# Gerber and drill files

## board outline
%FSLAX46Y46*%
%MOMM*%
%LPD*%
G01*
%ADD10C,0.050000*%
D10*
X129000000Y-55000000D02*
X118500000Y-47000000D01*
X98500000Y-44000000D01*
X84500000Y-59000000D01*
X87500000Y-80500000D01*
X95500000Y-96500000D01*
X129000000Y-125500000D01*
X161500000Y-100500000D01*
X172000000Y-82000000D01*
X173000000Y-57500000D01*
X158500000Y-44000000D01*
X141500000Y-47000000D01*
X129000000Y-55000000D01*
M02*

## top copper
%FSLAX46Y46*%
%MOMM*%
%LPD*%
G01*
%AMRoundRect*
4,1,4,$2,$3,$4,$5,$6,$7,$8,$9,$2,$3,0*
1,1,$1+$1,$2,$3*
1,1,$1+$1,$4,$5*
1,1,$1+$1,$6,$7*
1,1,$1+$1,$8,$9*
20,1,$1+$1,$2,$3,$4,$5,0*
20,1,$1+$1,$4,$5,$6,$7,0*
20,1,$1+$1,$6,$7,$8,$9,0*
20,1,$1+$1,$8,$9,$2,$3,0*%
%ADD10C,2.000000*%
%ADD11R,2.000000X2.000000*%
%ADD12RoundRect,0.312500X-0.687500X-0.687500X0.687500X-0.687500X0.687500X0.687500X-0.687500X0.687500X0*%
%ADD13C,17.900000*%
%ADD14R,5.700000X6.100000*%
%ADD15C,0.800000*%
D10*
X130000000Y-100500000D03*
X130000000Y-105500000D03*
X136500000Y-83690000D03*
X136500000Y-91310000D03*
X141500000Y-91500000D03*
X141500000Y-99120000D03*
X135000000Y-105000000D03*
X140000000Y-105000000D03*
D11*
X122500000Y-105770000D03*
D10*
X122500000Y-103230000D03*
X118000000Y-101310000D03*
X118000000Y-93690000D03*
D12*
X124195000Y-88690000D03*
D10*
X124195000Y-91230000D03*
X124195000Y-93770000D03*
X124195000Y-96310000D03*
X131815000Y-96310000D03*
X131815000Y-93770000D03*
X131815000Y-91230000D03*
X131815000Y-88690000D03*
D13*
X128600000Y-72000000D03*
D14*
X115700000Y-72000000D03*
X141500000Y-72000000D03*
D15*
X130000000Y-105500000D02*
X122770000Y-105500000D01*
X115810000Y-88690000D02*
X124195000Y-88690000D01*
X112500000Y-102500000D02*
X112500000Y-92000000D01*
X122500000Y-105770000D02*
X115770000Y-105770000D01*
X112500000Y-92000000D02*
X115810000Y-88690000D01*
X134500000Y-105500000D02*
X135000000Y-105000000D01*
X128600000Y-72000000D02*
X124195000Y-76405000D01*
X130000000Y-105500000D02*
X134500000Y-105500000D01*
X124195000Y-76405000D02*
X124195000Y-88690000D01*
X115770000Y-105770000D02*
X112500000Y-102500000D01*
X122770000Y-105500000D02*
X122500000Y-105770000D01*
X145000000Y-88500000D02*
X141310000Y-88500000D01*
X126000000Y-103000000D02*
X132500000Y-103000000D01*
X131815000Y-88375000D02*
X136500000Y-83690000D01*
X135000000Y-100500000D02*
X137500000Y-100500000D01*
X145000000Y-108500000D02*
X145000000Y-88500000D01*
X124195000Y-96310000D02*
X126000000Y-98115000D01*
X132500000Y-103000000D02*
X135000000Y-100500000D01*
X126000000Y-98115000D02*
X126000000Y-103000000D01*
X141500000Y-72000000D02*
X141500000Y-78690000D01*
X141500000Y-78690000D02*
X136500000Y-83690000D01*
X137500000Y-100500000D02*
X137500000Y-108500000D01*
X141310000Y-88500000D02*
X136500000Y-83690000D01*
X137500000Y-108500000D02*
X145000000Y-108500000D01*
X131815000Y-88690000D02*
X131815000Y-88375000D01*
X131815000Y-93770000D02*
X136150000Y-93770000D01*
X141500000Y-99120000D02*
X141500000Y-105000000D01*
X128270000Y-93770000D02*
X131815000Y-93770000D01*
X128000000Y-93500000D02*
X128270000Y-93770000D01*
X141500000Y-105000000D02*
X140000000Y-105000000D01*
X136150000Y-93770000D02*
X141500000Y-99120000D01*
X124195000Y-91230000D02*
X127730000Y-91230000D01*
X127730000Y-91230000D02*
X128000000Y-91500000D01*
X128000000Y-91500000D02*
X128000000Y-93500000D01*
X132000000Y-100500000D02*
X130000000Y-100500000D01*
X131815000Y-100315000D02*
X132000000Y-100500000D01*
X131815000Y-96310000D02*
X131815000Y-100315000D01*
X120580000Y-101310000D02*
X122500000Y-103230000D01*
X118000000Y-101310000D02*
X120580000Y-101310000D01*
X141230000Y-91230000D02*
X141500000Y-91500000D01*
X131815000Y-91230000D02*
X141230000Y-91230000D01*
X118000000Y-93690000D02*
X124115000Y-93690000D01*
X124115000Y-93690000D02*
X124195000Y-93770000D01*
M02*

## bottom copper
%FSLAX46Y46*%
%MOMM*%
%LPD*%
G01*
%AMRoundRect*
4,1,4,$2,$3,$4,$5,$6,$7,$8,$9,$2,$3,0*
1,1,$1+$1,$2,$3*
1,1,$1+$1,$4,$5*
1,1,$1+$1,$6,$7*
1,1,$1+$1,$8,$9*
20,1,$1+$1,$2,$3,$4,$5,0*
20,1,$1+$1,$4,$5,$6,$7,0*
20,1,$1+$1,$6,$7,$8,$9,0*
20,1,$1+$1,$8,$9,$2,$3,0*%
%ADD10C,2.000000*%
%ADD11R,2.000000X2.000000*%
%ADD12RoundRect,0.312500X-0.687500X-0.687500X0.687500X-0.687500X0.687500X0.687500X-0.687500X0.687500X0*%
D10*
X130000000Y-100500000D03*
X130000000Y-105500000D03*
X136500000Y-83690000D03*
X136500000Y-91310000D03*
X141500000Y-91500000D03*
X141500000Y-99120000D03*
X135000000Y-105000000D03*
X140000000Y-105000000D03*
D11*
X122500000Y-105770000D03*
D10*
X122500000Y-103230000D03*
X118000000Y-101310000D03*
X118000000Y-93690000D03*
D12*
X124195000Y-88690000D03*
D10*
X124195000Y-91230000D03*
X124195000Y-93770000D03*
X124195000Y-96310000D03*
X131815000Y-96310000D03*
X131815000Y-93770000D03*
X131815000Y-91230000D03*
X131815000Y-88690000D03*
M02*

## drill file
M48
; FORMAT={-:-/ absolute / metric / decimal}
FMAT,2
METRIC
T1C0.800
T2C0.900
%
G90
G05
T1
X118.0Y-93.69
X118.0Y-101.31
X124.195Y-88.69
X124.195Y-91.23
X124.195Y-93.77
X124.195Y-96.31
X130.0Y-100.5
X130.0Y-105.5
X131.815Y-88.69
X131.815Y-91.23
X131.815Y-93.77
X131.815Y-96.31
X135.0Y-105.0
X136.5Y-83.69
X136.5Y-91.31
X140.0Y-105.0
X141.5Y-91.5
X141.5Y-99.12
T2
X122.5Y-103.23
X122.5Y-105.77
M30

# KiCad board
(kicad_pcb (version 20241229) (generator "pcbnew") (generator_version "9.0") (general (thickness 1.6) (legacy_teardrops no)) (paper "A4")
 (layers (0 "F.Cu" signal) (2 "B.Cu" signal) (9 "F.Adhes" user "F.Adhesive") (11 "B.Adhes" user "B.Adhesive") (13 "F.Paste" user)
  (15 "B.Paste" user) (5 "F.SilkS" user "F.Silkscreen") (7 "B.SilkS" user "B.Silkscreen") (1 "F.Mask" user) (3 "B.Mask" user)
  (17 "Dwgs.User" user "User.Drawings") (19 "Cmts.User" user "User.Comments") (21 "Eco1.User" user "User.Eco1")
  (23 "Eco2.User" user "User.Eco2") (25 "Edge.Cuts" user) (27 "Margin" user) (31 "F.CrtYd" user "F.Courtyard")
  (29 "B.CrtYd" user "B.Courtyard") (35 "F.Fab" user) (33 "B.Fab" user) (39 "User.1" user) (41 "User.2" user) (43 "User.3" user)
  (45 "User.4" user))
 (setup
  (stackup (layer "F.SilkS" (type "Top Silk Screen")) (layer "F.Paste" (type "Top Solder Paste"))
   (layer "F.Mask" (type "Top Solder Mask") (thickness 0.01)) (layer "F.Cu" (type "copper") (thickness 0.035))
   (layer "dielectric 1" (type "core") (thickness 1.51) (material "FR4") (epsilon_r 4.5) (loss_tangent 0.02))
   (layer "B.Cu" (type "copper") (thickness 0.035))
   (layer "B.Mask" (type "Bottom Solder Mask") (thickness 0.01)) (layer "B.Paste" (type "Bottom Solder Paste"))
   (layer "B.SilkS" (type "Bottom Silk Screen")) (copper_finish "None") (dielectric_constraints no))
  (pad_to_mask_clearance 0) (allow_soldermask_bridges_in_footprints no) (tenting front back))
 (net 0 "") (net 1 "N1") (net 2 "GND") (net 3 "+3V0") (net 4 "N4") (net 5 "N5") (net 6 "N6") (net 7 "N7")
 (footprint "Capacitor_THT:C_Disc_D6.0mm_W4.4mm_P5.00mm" (layer "F.Cu") (at 130 100.5 -90)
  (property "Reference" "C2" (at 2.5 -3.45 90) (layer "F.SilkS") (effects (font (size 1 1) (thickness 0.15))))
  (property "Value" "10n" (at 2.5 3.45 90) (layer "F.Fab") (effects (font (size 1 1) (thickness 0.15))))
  (pad "1" thru_hole circle (at 0 0 270) (size 2 2) (drill 0.8) (layers "*.Cu" "*.Mask") (remove_unused_layers no) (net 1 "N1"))
  (pad "2" thru_hole circle (at 5 0 270) (size 2 2) (drill 0.8) (layers "*.Cu" "*.Mask") (remove_unused_layers no) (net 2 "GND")))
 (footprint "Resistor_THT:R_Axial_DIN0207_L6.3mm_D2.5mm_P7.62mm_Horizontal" (layer "F.Cu") (at 136.5 83.69 -90)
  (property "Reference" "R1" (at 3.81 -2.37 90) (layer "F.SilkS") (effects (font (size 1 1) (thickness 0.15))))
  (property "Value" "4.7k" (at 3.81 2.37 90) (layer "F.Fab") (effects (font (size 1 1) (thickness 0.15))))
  (pad "1" thru_hole circle (at 0 0 270) (size 2 2) (drill 0.8) (layers "*.Cu" "*.Mask") (remove_unused_layers no) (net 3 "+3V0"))
  (pad "2" thru_hole circle (at 7.62 0 270) (size 2 2) (drill 0.8) (layers "*.Cu" "*.Mask") (remove_unused_layers no) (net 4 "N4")))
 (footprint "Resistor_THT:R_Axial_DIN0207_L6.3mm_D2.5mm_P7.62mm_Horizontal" (layer "F.Cu") (at 141.5 91.5 -90)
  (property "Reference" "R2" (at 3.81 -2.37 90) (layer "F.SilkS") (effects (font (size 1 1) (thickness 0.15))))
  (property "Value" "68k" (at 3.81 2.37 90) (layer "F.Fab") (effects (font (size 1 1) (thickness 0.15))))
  (pad "1" thru_hole circle (at 0 0 270) (size 2 2) (drill 0.8) (layers "*.Cu" "*.Mask") (remove_unused_layers no) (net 4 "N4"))
  (pad "2" thru_hole circle (at 7.62 0 270) (size 2 2) (drill 0.8) (layers "*.Cu" "*.Mask") (remove_unused_layers no) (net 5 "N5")))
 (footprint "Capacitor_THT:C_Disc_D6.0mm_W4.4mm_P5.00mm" (layer "F.Cu") (at 135 105)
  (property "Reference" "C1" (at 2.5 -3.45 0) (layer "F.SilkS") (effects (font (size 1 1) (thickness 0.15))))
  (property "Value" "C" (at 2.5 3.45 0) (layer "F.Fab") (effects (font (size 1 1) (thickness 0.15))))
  (pad "1" thru_hole circle (at 0 0) (size 2 2) (drill 0.8) (layers "*.Cu" "*.Mask") (remove_unused_layers no) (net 2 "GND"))
  (pad "2" thru_hole circle (at 5 0) (size 2 2) (drill 0.8) (layers "*.Cu" "*.Mask") (remove_unused_layers no) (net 5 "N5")))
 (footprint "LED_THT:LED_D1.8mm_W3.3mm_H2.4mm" (layer "F.Cu") (at 122.5 105.77 90)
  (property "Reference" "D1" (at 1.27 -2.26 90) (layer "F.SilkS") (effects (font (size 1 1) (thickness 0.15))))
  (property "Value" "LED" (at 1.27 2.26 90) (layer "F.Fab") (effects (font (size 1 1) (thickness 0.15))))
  (pad "1" thru_hole rect (at 0 0 90) (size 2 2) (drill 0.9) (layers "*.Cu" "*.Mask") (remove_unused_layers no) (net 2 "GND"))
  (pad "2" thru_hole circle (at 2.54 0 90) (size 2 2) (drill 0.9) (layers "*.Cu" "*.Mask") (remove_unused_layers no) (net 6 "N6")))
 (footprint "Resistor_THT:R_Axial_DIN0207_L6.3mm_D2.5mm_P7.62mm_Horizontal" (layer "F.Cu") (at 118 101.31 90)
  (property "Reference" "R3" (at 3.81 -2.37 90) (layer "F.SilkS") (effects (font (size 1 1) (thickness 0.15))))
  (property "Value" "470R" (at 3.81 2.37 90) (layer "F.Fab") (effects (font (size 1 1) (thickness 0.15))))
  (pad "1" thru_hole circle (at 0 0 90) (size 2 2) (drill 0.8) (layers "*.Cu" "*.Mask") (remove_unused_layers no) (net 6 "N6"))
  (pad "2" thru_hole circle (at 7.62 0 90) (size 2 2) (drill 0.8) (layers "*.Cu" "*.Mask") (remove_unused_layers no) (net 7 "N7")))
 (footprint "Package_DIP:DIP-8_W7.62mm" (layer "F.Cu") (at 124.195 88.69)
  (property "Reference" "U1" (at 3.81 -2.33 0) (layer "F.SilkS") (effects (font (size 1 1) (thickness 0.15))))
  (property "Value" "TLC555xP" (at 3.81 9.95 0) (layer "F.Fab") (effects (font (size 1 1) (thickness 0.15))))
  (pad "1" thru_hole roundrect (at 0 0) (size 2 2) (drill 0.8) (layers "*.Cu" "*.Mask") (remove_unused_layers no) (roundrect_rratio 0.15625)
   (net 2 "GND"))
  (pad "2" thru_hole circle (at 0 2.54) (size 2 2) (drill 0.8) (layers "*.Cu" "*.Mask") (remove_unused_layers no) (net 5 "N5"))
  (pad "3" thru_hole circle (at 0 5.08) (size 2 2) (drill 0.8) (layers "*.Cu" "*.Mask") (remove_unused_layers no) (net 7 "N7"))
  (pad "4" thru_hole circle (at 0 7.62) (size 2 2) (drill 0.8) (layers "*.Cu" "*.Mask") (remove_unused_layers no) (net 3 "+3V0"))
  (pad "5" thru_hole circle (at 7.62 7.62) (size 2 2) (drill 0.8) (layers "*.Cu" "*.Mask") (remove_unused_layers no) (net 1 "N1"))
  (pad "6" thru_hole circle (at 7.62 5.08) (size 2 2) (drill 0.8) (layers "*.Cu" "*.Mask") (remove_unused_layers no) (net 5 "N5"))
  (pad "7" thru_hole circle (at 7.62 2.54) (size 2 2) (drill 0.8) (layers "*.Cu" "*.Mask") (remove_unused_layers no) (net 4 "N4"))
  (pad "8" thru_hole circle (at 7.62 0) (size 2 2) (drill 0.8) (layers "*.Cu" "*.Mask") (remove_unused_layers no) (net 3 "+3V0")))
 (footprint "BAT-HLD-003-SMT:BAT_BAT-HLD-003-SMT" (layer "F.Cu") (at 128.6 72)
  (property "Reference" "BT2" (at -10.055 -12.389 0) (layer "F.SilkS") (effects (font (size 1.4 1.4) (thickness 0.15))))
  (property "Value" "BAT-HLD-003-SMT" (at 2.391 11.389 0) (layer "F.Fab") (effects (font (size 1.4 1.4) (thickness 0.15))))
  (pad "N" smd circle (at 0 0) (size 17.9 17.9) (layers "F.Cu" "F.Mask") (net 2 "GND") (solder_mask_margin 0.102))
  (pad "P1" smd rect (at -12.9 0) (size 5.7 6.1) (layers "F.Cu" "F.Mask" "F.Paste") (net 3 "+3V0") (solder_mask_margin 0.102))
  (pad "P2" smd rect (at 12.9 0) (size 5.7 6.1) (layers "F.Cu" "F.Mask" "F.Paste") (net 3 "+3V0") (solder_mask_margin 0.102)))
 (gr_poly
  (pts (xy 129 55) (xy 118.5 47) (xy 98.5 44) (xy 84.5 59) (xy 87.5 80.5) (xy 95.5 96.5) (xy 129 125.5) (xy 161.5 100.5) (xy 172 82)
   (xy 173 57.5) (xy 158.5 44) (xy 141.5 47))
  (stroke (width 0.05) (type solid)) (fill no) (layer "Edge.Cuts"))
 (segment (start 130 105.5) (end 122.77 105.5) (width 0.8) (layer "F.Cu") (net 2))
 (segment (start 115.81 88.69) (end 124.195 88.69) (width 0.8) (layer "F.Cu") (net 2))
 (segment (start 112.5 102.5) (end 112.5 92) (width 0.8) (layer "F.Cu") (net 2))
 (segment (start 122.5 105.77) (end 115.77 105.77) (width 0.8) (layer "F.Cu") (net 2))
 (segment (start 112.5 92) (end 115.81 88.69) (width 0.8) (layer "F.Cu") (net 2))
 (segment (start 134.5 105.5) (end 135 105) (width 0.8) (layer "F.Cu") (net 2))
 (segment (start 128.6 72) (end 124.195 76.405) (width 0.8) (layer "F.Cu") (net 2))
 (segment (start 130 105.5) (end 134.5 105.5) (width 0.8) (layer "F.Cu") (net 2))
 (segment (start 124.195 76.405) (end 124.195 88.69) (width 0.8) (layer "F.Cu") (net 2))
 (segment (start 115.77 105.77) (end 112.5 102.5) (width 0.8) (layer "F.Cu") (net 2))
 (segment (start 122.77 105.5) (end 122.5 105.77) (width 0.8) (layer "F.Cu") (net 2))
 (segment (start 145 88.5) (end 141.31 88.5) (width 0.8) (layer "F.Cu") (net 3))
 (segment (start 126 103) (end 132.5 103) (width 0.8) (layer "F.Cu") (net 3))
 (segment (start 131.815 88.375) (end 136.5 83.69) (width 0.8) (layer "F.Cu") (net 3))
 (segment (start 135 100.5) (end 137.5 100.5) (width 0.8) (layer "F.Cu") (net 3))
 (segment (start 145 108.5) (end 145 88.5) (width 0.8) (layer "F.Cu") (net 3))
 (segment (start 124.195 96.31) (end 126 98.115) (width 0.8) (layer "F.Cu") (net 3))
 (segment (start 132.5 103) (end 135 100.5) (width 0.8) (layer "F.Cu") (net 3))
 (segment (start 126 98.115) (end 126 103) (width 0.8) (layer "F.Cu") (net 3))
 (segment (start 141.5 72) (end 141.5 78.69) (width 0.8) (layer "F.Cu") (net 3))
 (segment (start 141.5 78.69) (end 136.5 83.69) (width 0.8) (layer "F.Cu") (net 3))
 (segment (start 137.5 100.5) (end 137.5 108.5) (width 0.8) (layer "F.Cu") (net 3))
 (segment (start 141.31 88.5) (end 136.5 83.69) (width 0.8) (layer "F.Cu") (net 3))
 (segment (start 137.5 108.5) (end 145 108.5) (width 0.8) (layer "F.Cu") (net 3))
 (segment (start 131.815 88.69) (end 131.815 88.375) (width 0.8) (layer "F.Cu") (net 3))
 (segment (start 131.815 93.77) (end 136.15 93.77) (width 0.8) (layer "F.Cu") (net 5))
 (segment (start 141.5 99.12) (end 141.5 105) (width 0.8) (layer "F.Cu") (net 5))
 (segment (start 128.27 93.77) (end 131.815 93.77) (width 0.8) (layer "F.Cu") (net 5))
 (segment (start 128 93.5) (end 128.27 93.77) (width 0.8) (layer "F.Cu") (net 5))
 (segment (start 141.5 105) (end 140 105) (width 0.8) (layer "F.Cu") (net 5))
 (segment (start 136.15 93.77) (end 141.5 99.12) (width 0.8) (layer "F.Cu") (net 5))
 (segment (start 124.195 91.23) (end 127.73 91.23) (width 0.8) (layer "F.Cu") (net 5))
 (segment (start 127.73 91.23) (end 128 91.5) (width 0.8) (layer "F.Cu") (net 5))
 (segment (start 128 91.5) (end 128 93.5) (width 0.8) (layer "F.Cu") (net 5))
 (segment (start 132 100.5) (end 130 100.5) (width 0.8) (layer "F.Cu") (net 1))
 (segment (start 131.815 100.315) (end 132 100.5) (width 0.8) (layer "F.Cu") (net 1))
 (segment (start 131.815 96.31) (end 131.815 100.315) (width 0.8) (layer "F.Cu") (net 1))
 (segment (start 120.58 101.31) (end 122.5 103.23) (width 0.8) (layer "F.Cu") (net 6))
 (segment (start 118 101.31) (end 120.58 101.31) (width 0.8) (layer "F.Cu") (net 6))
 (segment (start 141.23 91.23) (end 141.5 91.5) (width 0.8) (layer "F.Cu") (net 4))
 (segment (start 131.815 91.23) (end 141.23 91.23) (width 0.8) (layer "F.Cu") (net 4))
 (segment (start 118 93.69) (end 124.115 93.69) (width 0.8) (layer "F.Cu") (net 7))
 (segment (start 124.115 93.69) (end 124.195 93.77) (width 0.8) (layer "F.Cu") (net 7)))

